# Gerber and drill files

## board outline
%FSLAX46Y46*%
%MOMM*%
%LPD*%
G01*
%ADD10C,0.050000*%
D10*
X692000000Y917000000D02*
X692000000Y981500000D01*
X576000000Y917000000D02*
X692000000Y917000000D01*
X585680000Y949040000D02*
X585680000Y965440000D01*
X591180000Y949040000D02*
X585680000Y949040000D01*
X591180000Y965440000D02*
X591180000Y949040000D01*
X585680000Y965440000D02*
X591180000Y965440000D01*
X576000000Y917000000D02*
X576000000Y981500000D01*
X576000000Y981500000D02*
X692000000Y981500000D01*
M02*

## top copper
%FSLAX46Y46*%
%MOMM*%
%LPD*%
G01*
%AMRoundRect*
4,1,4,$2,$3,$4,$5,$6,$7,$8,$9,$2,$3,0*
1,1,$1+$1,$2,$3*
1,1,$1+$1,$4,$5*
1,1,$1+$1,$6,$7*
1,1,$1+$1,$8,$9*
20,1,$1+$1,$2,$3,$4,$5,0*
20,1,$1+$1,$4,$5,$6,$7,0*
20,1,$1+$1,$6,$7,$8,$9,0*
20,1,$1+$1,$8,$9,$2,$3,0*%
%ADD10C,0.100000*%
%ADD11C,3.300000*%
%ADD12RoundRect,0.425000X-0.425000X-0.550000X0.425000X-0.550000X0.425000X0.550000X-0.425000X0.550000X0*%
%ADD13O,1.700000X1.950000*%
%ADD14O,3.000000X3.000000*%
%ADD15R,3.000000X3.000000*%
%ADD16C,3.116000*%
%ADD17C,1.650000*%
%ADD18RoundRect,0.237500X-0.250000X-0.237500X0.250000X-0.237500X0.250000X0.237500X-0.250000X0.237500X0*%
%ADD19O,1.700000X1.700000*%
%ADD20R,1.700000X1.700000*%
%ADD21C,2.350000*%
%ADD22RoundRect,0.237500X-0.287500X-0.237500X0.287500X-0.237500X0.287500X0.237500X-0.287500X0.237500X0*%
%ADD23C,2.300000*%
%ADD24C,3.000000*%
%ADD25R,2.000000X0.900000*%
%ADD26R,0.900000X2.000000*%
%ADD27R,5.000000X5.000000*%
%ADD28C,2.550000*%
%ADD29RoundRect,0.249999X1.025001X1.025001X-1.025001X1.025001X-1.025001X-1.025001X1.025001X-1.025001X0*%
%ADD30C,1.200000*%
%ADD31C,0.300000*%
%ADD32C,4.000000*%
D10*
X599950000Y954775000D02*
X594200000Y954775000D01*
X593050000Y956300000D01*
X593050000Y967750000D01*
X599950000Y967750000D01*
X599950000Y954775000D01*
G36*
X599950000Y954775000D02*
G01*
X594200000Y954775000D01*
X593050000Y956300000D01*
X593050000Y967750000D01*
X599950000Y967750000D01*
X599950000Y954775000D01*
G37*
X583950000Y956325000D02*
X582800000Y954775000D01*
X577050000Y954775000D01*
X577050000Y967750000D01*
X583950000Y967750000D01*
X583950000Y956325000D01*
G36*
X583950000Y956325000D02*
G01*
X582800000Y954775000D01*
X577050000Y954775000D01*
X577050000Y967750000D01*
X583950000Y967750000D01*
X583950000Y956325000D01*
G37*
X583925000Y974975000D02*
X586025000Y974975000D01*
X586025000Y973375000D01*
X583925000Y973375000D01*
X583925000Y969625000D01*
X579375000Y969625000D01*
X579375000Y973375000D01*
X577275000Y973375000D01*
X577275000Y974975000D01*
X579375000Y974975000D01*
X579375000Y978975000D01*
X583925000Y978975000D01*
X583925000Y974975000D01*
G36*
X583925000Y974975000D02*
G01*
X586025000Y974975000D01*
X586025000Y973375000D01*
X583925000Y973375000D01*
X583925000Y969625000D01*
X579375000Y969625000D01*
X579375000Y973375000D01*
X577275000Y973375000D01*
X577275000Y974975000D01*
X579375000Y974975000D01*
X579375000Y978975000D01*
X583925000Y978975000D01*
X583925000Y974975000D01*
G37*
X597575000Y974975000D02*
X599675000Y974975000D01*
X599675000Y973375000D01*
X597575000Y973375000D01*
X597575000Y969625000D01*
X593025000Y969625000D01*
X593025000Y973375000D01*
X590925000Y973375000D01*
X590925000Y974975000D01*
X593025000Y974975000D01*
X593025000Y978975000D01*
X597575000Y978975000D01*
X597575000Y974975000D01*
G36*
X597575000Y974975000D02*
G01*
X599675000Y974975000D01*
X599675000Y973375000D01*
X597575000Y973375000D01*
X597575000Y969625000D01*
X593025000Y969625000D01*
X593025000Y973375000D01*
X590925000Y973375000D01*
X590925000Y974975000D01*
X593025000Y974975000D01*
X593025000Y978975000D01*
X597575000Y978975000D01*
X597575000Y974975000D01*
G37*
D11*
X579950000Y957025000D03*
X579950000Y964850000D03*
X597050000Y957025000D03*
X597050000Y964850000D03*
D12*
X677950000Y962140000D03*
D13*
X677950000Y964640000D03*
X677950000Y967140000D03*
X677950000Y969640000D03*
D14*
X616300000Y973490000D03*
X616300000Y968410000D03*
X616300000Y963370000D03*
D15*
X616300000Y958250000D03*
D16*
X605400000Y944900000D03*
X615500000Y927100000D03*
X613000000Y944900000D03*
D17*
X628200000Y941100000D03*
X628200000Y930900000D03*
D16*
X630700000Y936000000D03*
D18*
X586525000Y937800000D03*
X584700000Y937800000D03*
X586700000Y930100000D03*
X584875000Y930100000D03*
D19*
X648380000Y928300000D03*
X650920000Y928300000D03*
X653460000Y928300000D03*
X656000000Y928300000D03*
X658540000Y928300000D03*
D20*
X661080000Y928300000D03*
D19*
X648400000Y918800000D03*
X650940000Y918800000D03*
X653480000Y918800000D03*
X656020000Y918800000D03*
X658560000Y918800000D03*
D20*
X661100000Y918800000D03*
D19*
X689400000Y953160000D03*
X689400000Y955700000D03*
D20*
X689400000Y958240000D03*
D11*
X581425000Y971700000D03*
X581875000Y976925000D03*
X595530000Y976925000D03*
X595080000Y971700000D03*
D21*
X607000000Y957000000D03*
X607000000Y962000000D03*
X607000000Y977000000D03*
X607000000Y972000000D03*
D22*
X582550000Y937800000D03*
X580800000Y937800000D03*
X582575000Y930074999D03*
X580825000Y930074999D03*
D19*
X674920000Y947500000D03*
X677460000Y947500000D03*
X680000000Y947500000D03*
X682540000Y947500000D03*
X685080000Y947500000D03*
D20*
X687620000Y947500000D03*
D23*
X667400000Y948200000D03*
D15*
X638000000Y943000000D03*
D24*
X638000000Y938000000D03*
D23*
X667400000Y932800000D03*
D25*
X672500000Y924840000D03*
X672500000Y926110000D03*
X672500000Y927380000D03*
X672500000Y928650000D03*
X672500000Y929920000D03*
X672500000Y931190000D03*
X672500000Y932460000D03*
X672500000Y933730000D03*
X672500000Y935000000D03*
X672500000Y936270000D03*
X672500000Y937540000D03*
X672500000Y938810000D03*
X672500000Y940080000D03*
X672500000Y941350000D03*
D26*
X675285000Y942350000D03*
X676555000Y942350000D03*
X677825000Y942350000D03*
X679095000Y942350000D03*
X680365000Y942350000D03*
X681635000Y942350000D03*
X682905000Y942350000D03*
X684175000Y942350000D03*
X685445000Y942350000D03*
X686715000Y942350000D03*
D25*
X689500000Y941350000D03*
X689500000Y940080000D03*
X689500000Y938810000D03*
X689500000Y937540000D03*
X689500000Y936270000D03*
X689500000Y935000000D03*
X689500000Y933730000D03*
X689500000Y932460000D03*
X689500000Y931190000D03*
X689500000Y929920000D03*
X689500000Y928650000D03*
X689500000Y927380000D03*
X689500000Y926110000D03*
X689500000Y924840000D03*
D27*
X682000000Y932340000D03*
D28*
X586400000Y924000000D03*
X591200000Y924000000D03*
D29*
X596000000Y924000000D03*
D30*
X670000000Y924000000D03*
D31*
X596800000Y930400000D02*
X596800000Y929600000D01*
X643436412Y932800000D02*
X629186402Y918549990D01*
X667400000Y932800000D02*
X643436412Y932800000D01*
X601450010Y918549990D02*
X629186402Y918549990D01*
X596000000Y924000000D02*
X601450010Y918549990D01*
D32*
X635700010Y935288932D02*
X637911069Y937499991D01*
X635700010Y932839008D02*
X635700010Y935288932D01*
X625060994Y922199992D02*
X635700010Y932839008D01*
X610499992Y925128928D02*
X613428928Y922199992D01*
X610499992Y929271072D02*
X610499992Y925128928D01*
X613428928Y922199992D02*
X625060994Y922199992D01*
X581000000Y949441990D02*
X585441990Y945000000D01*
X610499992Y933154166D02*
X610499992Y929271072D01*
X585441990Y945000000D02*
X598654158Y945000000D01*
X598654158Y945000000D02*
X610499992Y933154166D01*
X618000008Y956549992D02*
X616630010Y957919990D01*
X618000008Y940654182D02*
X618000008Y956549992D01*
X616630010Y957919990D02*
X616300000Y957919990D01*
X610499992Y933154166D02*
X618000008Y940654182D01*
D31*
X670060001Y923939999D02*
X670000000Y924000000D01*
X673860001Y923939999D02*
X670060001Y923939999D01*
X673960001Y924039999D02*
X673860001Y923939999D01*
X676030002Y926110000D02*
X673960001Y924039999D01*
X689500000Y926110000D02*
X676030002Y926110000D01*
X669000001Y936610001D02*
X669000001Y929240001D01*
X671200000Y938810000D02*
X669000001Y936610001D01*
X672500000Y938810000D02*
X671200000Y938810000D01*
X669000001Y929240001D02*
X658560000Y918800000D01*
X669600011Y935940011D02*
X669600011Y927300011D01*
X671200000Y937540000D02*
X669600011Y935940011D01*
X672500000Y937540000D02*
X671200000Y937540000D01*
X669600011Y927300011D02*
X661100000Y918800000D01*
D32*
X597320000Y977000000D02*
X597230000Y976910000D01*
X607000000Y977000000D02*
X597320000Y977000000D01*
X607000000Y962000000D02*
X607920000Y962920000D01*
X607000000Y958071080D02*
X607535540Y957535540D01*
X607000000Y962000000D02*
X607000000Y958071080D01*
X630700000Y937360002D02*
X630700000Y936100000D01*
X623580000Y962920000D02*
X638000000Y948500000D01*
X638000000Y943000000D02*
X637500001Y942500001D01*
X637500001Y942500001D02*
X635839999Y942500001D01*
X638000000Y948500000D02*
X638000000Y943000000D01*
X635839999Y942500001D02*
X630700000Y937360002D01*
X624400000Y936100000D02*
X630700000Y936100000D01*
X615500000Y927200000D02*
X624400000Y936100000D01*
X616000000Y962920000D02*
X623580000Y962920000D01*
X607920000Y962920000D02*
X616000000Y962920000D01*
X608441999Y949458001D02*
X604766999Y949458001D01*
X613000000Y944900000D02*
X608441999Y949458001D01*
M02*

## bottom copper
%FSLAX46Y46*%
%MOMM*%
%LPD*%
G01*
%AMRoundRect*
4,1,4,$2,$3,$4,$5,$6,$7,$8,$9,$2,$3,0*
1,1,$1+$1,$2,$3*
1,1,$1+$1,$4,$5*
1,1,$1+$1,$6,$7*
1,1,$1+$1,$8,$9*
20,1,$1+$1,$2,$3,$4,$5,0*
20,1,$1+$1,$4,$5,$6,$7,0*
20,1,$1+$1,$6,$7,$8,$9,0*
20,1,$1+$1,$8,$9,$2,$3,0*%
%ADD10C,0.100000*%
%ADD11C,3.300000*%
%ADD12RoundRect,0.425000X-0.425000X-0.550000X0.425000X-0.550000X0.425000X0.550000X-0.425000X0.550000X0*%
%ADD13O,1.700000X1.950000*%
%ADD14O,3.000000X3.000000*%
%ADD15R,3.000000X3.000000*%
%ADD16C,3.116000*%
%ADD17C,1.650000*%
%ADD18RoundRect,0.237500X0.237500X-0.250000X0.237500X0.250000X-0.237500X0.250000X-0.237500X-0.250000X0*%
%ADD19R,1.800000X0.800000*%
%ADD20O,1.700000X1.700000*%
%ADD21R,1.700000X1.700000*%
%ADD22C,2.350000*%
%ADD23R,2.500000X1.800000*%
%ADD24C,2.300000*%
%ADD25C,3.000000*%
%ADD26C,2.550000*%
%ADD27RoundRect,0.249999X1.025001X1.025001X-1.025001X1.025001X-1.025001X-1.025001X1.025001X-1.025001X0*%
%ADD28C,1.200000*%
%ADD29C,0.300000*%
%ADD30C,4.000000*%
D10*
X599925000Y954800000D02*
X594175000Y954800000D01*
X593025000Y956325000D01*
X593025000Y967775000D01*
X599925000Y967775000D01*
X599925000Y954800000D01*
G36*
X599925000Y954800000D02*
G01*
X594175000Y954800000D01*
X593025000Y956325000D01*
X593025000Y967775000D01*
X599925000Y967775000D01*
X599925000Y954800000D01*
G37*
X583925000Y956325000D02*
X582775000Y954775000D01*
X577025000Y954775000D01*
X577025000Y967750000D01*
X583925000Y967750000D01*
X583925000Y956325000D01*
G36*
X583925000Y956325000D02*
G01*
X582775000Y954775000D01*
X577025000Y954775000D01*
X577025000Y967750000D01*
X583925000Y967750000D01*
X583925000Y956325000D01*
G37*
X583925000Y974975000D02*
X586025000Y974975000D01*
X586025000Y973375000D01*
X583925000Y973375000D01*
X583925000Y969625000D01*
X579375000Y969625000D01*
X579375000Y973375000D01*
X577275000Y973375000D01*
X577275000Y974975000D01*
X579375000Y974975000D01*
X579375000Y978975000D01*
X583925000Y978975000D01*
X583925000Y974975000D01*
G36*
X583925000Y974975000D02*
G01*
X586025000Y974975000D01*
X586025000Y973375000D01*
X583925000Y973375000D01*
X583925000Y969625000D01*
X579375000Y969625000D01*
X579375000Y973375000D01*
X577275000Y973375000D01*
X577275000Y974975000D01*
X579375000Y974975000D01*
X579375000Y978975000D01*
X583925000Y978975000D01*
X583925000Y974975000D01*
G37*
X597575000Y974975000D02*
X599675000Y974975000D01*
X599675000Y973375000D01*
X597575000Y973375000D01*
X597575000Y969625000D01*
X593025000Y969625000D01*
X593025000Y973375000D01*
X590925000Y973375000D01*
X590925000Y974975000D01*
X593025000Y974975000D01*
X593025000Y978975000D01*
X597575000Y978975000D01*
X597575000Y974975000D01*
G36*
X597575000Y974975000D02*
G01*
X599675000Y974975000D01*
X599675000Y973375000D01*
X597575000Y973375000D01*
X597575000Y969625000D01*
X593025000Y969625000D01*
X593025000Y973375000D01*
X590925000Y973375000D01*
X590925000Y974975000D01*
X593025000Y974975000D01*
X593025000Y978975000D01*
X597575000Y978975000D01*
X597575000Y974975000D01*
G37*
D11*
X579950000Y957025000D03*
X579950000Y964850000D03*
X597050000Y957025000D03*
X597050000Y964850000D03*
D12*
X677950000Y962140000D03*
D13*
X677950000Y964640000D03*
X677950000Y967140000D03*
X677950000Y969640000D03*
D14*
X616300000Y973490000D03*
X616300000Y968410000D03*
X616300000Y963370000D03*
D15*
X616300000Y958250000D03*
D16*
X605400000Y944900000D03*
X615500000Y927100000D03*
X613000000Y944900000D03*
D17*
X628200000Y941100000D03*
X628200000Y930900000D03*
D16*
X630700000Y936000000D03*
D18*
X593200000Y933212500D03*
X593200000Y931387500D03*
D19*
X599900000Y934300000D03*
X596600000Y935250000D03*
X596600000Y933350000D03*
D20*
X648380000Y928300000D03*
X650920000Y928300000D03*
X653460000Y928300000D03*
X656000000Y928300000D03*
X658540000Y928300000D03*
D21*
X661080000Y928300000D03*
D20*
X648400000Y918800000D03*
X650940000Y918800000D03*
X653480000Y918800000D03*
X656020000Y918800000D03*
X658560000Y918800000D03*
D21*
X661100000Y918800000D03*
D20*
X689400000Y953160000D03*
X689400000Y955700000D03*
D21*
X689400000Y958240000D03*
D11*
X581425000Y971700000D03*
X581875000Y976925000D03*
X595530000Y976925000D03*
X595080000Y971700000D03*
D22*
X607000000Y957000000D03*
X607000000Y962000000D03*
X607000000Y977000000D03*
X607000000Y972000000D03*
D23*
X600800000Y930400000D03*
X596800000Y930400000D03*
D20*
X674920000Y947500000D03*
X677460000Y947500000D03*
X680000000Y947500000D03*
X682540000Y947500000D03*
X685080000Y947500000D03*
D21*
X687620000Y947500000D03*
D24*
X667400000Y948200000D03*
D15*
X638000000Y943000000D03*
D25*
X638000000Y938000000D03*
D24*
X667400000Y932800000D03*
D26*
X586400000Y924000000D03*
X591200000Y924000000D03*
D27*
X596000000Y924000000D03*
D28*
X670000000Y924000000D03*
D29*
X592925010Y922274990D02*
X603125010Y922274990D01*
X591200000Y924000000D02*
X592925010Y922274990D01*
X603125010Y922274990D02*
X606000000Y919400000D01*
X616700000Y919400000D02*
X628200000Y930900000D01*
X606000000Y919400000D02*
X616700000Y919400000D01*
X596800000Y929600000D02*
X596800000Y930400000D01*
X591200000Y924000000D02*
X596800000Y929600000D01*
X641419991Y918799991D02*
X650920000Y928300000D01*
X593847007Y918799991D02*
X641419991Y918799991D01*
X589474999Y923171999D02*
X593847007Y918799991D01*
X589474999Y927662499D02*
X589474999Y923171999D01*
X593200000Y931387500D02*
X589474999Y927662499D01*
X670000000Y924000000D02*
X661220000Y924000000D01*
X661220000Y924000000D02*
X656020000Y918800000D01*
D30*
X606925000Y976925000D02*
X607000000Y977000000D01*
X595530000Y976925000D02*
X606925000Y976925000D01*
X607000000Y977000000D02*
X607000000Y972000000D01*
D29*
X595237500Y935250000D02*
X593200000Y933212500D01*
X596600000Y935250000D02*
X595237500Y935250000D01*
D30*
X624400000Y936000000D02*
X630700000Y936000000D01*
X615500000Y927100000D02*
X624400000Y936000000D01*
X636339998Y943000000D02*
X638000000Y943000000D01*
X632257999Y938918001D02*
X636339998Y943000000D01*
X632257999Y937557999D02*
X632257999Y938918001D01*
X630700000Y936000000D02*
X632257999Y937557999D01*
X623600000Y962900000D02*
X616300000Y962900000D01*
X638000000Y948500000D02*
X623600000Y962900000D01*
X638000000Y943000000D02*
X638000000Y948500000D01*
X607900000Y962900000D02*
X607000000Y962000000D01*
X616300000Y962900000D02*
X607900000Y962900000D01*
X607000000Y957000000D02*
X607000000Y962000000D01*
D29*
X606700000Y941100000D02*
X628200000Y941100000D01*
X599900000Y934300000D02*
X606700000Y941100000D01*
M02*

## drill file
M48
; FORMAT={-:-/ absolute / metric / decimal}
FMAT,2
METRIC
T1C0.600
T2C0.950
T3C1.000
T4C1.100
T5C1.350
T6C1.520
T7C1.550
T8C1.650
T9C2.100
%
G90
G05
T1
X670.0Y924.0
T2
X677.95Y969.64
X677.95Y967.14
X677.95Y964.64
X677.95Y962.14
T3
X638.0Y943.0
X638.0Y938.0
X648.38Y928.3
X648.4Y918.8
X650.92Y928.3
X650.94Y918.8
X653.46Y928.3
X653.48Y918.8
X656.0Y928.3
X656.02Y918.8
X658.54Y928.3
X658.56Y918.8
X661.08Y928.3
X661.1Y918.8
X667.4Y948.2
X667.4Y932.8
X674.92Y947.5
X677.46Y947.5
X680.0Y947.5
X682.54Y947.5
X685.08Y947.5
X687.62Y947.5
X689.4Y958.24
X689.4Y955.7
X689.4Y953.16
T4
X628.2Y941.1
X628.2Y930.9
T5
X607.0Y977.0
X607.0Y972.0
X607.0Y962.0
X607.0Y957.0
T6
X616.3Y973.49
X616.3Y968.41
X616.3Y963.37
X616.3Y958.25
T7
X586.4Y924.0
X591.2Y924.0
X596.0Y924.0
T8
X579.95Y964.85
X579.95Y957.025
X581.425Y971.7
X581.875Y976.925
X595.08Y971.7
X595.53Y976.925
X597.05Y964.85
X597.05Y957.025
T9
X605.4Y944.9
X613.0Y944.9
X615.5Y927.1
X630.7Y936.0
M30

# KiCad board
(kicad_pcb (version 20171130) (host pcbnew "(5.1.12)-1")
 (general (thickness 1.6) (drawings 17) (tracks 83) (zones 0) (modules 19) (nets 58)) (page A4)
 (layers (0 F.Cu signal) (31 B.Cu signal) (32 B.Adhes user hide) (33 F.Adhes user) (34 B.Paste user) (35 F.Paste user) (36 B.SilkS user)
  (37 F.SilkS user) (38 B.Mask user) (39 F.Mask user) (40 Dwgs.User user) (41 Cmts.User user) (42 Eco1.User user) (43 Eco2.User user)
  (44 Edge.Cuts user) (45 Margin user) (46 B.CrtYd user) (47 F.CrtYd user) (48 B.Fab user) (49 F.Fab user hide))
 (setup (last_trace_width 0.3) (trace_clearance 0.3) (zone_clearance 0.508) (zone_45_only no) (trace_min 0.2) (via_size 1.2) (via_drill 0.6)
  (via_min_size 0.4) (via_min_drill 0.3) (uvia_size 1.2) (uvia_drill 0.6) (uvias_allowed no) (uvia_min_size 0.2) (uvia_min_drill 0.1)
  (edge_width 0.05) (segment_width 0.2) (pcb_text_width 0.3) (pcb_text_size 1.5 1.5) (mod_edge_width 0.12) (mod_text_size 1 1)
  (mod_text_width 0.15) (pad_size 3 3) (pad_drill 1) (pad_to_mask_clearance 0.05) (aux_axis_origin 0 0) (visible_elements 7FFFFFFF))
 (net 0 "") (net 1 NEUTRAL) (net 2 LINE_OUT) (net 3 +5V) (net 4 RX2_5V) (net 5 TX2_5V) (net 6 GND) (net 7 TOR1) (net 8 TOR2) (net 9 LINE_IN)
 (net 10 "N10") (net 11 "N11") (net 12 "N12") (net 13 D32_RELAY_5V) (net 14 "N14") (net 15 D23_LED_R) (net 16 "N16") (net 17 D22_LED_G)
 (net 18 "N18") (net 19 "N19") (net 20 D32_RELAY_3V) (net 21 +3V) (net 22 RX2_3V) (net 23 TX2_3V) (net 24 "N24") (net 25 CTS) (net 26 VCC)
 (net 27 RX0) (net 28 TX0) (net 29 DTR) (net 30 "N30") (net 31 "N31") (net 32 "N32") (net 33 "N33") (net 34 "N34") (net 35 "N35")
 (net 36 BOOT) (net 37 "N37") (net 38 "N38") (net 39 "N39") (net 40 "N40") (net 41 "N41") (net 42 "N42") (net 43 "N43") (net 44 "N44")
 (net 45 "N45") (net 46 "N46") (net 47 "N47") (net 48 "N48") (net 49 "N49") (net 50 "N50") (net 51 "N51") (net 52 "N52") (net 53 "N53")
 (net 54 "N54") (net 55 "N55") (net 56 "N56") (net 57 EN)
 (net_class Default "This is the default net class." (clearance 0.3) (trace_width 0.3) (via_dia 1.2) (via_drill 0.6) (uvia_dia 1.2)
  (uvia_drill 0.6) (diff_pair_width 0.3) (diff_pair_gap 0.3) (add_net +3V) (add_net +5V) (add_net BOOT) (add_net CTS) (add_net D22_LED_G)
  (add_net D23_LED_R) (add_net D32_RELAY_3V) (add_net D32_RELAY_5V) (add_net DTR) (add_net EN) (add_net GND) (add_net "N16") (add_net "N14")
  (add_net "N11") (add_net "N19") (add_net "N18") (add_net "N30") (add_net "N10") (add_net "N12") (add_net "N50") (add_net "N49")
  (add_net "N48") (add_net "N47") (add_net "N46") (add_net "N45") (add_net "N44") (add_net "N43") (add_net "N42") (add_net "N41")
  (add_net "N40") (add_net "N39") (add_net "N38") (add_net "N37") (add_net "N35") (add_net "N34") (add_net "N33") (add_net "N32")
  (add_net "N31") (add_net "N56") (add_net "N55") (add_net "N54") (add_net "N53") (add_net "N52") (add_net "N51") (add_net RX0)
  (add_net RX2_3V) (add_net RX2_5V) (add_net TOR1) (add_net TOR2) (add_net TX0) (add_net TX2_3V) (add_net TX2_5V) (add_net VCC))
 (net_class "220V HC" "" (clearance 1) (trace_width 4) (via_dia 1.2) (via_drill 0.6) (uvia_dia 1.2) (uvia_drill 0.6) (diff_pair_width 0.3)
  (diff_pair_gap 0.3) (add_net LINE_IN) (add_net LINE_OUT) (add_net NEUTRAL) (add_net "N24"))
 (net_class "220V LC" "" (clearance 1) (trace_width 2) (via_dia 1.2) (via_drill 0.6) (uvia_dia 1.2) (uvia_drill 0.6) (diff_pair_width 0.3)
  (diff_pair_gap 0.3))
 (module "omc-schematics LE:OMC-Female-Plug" (layer F.Cu) (at 588.5 -962.1)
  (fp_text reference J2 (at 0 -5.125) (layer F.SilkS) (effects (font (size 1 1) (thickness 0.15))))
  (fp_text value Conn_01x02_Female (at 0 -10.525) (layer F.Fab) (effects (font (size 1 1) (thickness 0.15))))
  (fp_poly (pts (xy 11.425 7.3) (xy 5.675 7.3) (xy 4.525 5.775) (xy 4.525 -5.675) (xy 11.425 -5.675)) (layer B.Cu) (width 0.1))
  (fp_poly (pts (xy 11.45 7.325) (xy 5.7 7.325) (xy 4.55 5.8) (xy 4.55 -5.65) (xy 11.45 -5.65)) (layer F.Cu) (width 0.1))
  (fp_poly (pts (xy -4.575 5.775) (xy -5.725 7.325) (xy -11.475 7.325) (xy -11.475 -5.65) (xy -4.575 -5.65)) (layer B.Cu) (width 0.1))
  (fp_poly (pts (xy -4.55 5.775) (xy -5.7 7.325) (xy -11.45 7.325) (xy -11.45 -5.65) (xy -4.55 -5.65)) (layer F.Cu) (width 0.1))
  (pad 1 thru_hole circle (at -8.55 5.075) (size 3.3 3.3) (drill 1.65) (layers *.Cu *.Mask) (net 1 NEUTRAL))
  (pad 1 thru_hole circle (at -8.55 -2.75) (size 3.3 3.3) (drill 1.65) (layers *.Cu *.Mask) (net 1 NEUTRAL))
  (pad 2 thru_hole circle (at 8.55 5.075) (size 3.3 3.3) (drill 1.65) (layers *.Cu *.Mask) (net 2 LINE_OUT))
  (pad 2 thru_hole circle (at 8.55 -2.75) (size 3.3 3.3) (drill 1.65) (layers *.Cu *.Mask) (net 2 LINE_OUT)))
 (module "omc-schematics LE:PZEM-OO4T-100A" (layer F.Cu) (at 649.18 -965.9)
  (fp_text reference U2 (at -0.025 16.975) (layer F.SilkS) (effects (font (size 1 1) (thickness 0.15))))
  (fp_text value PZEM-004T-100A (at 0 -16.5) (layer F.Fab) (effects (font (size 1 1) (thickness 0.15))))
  (pad 5 thru_hole roundrect (at 28.77 3.76) (size 1.7 1.95) (drill 0.95) (layers *.Cu *.Mask) (roundrect_rratio 0.25) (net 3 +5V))
  (pad 6 thru_hole oval (at 28.77 1.26) (size 1.7 1.95) (drill 0.95) (layers *.Cu *.Mask) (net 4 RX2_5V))
  (pad 7 thru_hole oval (at 28.77 -1.24) (size 1.7 1.95) (drill 0.95) (layers *.Cu *.Mask) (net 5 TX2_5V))
  (pad 8 thru_hole oval (at 28.77 -3.74) (size 1.7 1.95) (drill 0.95) (layers *.Cu *.Mask) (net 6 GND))
  (pad 4 thru_hole oval (at -32.88 -7.59) (size 3 3) (drill 1.52) (layers *.Cu *.Mask) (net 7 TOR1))
  (pad 3 thru_hole oval (at -32.88 -2.51) (size 3 3) (drill 1.52) (layers *.Cu *.Mask) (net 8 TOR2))
  (pad 2 thru_hole oval (at -32.88 2.53) (size 3 3) (drill 1.52) (layers *.Cu *.Mask) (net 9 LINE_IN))
  (pad 1 thru_hole rect (at -32.88 7.65) (size 3 3) (drill 1.52) (layers *.Cu *.Mask) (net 1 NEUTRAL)))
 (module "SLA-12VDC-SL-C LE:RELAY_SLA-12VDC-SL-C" (layer F.Cu) (at 613 -936 90)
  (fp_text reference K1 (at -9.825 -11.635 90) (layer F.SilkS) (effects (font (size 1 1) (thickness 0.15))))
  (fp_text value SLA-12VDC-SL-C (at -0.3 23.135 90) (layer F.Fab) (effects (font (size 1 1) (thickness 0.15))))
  (pad NC thru_hole circle (at 8.9 -7.6 90) (size 3.116 3.116) (drill 2.1) (layers *.Cu *.Mask) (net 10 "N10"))
  (pad COM2 thru_hole circle (at -8.9 2.5 90) (size 3.116 3.116) (drill 2.1) (layers *.Cu *.Mask) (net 9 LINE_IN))
  (pad NO thru_hole circle (at 8.9 0 90) (size 3.116 3.116) (drill 2.1) (layers *.Cu *.Mask) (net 2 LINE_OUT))
  (pad C2 thru_hole circle (at 5.1 15.2 90) (size 1.65 1.65) (drill 1.1) (layers *.Cu *.Mask) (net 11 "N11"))
  (pad C1 thru_hole circle (at -5.1 15.2 90) (size 1.65 1.65) (drill 1.1) (layers *.Cu *.Mask) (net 3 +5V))
  (pad COM1 thru_hole circle (at 0 17.7 90) (size 3.116 3.116) (drill 2.1) (layers *.Cu *.Mask) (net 9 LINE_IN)))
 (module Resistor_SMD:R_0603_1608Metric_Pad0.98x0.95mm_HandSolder (layer B.Cu) (at 593.2 -932.3 90)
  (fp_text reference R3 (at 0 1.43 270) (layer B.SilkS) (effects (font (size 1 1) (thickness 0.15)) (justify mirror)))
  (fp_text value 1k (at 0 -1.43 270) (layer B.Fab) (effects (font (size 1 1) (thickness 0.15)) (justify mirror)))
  (pad 2 smd roundrect (at 0.9125 0 90) (size 0.975 0.95) (layers B.Cu B.Paste B.Mask) (roundrect_rratio 0.25) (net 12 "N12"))
  (pad 1 smd roundrect (at -0.9125 0 90) (size 0.975 0.95) (layers B.Cu B.Paste B.Mask) (roundrect_rratio 0.25) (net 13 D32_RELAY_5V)))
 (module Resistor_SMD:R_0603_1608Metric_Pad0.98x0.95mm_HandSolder (layer F.Cu) (at 585.6125 -937.8)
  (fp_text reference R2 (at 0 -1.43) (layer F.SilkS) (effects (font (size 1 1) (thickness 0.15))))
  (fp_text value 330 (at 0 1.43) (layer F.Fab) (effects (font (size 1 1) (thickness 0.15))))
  (pad 2 smd roundrect (at 0.9125 0) (size 0.975 0.95) (layers F.Cu F.Paste F.Mask) (roundrect_rratio 0.25) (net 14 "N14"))
  (pad 1 smd roundrect (at -0.9125 0) (size 0.975 0.95) (layers F.Cu F.Paste F.Mask) (roundrect_rratio 0.25) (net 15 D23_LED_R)))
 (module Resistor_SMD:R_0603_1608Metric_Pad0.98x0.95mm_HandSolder (layer F.Cu) (at 585.7875 -930.1)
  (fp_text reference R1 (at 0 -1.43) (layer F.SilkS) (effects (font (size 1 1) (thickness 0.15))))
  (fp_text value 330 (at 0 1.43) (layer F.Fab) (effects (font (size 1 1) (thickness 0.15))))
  (pad 2 smd roundrect (at 0.9125 0) (size 0.975 0.95) (layers F.Cu F.Paste F.Mask) (roundrect_rratio 0.25) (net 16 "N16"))
  (pad 1 smd roundrect (at -0.9125 0) (size 0.975 0.95) (layers F.Cu F.Paste F.Mask) (roundrect_rratio 0.25) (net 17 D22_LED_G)))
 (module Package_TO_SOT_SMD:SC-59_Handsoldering (layer B.Cu) (at 598.25 -934.3)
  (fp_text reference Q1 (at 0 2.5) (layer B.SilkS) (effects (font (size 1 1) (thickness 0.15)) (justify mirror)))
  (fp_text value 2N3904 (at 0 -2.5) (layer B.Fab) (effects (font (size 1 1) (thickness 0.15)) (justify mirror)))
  (pad 3 smd rect (at 1.65 0) (size 1.8 0.8) (layers B.Cu B.Paste B.Mask) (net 11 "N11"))
  (pad 2 smd rect (at -1.65 -0.95) (size 1.8 0.8) (layers B.Cu B.Paste B.Mask) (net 12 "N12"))
  (pad 1 smd rect (at -1.65 0.95) (size 1.8 0.8) (layers B.Cu B.Paste B.Mask) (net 6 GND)))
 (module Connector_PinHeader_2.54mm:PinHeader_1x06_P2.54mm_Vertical (layer F.Cu) (at 661.08 -928.3 270)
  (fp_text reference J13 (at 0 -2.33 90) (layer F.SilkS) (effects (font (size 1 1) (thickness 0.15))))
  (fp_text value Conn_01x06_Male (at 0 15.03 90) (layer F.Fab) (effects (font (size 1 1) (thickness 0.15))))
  (pad 6 thru_hole oval (at 0 12.7 270) (size 1.7 1.7) (drill 1) (layers *.Cu *.Mask) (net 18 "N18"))
  (pad 5 thru_hole oval (at 0 10.16 270) (size 1.7 1.7) (drill 1) (layers *.Cu *.Mask) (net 13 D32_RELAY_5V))
  (pad 4 thru_hole oval (at 0 7.62 270) (size 1.7 1.7) (drill 1) (layers *.Cu *.Mask) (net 6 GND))
  (pad 3 thru_hole oval (at 0 5.08 270) (size 1.7 1.7) (drill 1) (layers *.Cu *.Mask) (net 3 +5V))
  (pad 2 thru_hole oval (at 0 2.54 270) (size 1.7 1.7) (drill 1) (layers *.Cu *.Mask) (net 5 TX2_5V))
  (pad 1 thru_hole rect (at 0 0 270) (size 1.7 1.7) (drill 1) (layers *.Cu *.Mask) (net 4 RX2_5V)))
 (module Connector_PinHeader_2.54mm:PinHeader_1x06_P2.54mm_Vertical (layer F.Cu) (at 661.1 -918.8 270)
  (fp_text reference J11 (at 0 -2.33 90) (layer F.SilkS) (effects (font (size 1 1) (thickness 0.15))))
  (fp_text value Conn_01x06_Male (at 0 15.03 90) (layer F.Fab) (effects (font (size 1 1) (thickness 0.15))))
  (pad 6 thru_hole oval (at 0 12.7 270) (size 1.7 1.7) (drill 1) (layers *.Cu *.Mask) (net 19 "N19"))
  (pad 5 thru_hole oval (at 0 10.16 270) (size 1.7 1.7) (drill 1) (layers *.Cu *.Mask) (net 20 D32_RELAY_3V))
  (pad 4 thru_hole oval (at 0 7.62 270) (size 1.7 1.7) (drill 1) (layers *.Cu *.Mask) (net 6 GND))
  (pad 3 thru_hole oval (at 0 5.08 270) (size 1.7 1.7) (drill 1) (layers *.Cu *.Mask) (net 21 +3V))
  (pad 2 thru_hole oval (at 0 2.54 270) (size 1.7 1.7) (drill 1) (layers *.Cu *.Mask) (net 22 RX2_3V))
  (pad 1 thru_hole rect (at 0 0 270) (size 1.7 1.7) (drill 1) (layers *.Cu *.Mask) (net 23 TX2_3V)))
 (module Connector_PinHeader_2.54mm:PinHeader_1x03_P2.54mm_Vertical (layer F.Cu) (at 689.4 -958.24)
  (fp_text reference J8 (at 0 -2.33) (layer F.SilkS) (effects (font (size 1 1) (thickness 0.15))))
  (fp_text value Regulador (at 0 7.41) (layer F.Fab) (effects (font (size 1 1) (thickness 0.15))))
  (pad 3 thru_hole oval (at 0 5.08) (size 1.7 1.7) (drill 1) (layers *.Cu *.Mask) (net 3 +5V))
  (pad 2 thru_hole oval (at 0 2.54) (size 1.7 1.7) (drill 1) (layers *.Cu *.Mask) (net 21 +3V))
  (pad 1 thru_hole rect (at 0 0) (size 1.7 1.7) (drill 1) (layers *.Cu *.Mask) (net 6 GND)))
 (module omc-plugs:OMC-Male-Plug (layer F.Cu) (at 581.6 -974)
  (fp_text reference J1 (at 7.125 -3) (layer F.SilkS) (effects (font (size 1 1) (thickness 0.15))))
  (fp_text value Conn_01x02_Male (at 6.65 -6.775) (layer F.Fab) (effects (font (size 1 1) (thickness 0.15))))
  (fp_poly
   (pts (xy 2.325 -0.975) (xy 4.425 -0.975) (xy 4.425 0.625) (xy 2.325 0.625) (xy 2.325 4.375) (xy -2.225 4.375) (xy -2.225 0.625)
    (xy -4.325 0.625) (xy -4.325 -0.975) (xy -2.225 -0.975) (xy -2.225 -4.975) (xy 2.325 -4.975))
   (layer F.Cu) (width 0.1))
  (fp_poly
   (pts (xy 2.325 -0.975) (xy 4.425 -0.975) (xy 4.425 0.625) (xy 2.325 0.625) (xy 2.325 4.375) (xy -2.225 4.375) (xy -2.225 0.625)
    (xy -4.325 0.625) (xy -4.325 -0.975) (xy -2.225 -0.975) (xy -2.225 -4.975) (xy 2.325 -4.975))
   (layer B.Cu) (width 0.1))
  (fp_poly
   (pts (xy 15.975 -0.975) (xy 18.075 -0.975) (xy 18.075 0.625) (xy 15.975 0.625) (xy 15.975 4.375) (xy 11.425 4.375) (xy 11.425 0.625)
    (xy 9.325 0.625) (xy 9.325 -0.975) (xy 11.425 -0.975) (xy 11.425 -4.975) (xy 15.975 -4.975))
   (layer B.Cu) (width 0.1))
  (fp_poly
   (pts (xy 15.975 -0.975) (xy 18.075 -0.975) (xy 18.075 0.625) (xy 15.975 0.625) (xy 15.975 4.375) (xy 11.425 4.375) (xy 11.425 0.625)
    (xy 9.325 0.625) (xy 9.325 -0.975) (xy 11.425 -0.975) (xy 11.425 -4.975) (xy 15.975 -4.975))
   (layer F.Cu) (width 0.1))
  (pad 1 thru_hole circle (at -0.175 2.3) (size 3.3 3.3) (drill 1.65) (layers *.Cu *.Mask) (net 1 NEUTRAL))
  (pad 1 thru_hole circle (at 0.275 -2.925 270) (size 3.3 3.3) (drill 1.65) (layers *.Cu *.Mask) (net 1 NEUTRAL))
  (pad 2 thru_hole circle (at 13.93 -2.925 270) (size 3.3 3.3) (drill 1.65) (layers *.Cu *.Mask) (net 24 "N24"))
  (pad 2 thru_hole circle (at 13.48 2.3) (size 3.3 3.3) (drill 1.65) (layers *.Cu *.Mask) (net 24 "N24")))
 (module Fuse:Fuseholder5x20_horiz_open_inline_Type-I (layer F.Cu) (at 607 -957 90)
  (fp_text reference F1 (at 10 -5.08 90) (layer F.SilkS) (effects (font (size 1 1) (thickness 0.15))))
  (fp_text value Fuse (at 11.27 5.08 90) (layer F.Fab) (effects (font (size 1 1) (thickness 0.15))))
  (pad 1 thru_hole circle (at 0 0 90) (size 2.35 2.35) (drill 1.35) (layers *.Cu *.Mask) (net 9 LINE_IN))
  (pad 1 thru_hole circle (at 5 0 90) (size 2.35 2.35) (drill 1.35) (layers *.Cu *.Mask) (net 9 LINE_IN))
  (pad 2 thru_hole circle (at 20 0 90) (size 2.35 2.35) (drill 1.35) (layers *.Cu *.Mask) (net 24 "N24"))
  (pad 2 thru_hole circle (at 15 0 90) (size 2.35 2.35) (drill 1.35) (layers *.Cu *.Mask) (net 24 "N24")))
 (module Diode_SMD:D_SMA (layer B.Cu) (at 598.8 -930.4)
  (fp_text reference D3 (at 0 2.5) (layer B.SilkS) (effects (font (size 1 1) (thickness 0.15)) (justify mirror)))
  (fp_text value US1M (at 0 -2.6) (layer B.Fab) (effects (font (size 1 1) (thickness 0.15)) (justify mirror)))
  (pad 2 smd rect (at 2 0) (size 2.5 1.8) (layers B.Cu B.Paste B.Mask) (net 11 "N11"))
  (pad 1 smd rect (at -2 0) (size 2.5 1.8) (layers B.Cu B.Paste B.Mask) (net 3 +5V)))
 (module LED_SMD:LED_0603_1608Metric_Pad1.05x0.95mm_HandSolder (layer F.Cu) (at 581.675 -937.8)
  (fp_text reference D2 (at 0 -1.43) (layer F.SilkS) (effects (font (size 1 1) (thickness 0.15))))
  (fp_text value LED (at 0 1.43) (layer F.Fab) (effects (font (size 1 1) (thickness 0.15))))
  (pad 2 smd roundrect (at 0.875 0) (size 1.05 0.95) (layers F.Cu F.Paste F.Mask) (roundrect_rratio 0.25) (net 14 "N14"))
  (pad 1 smd roundrect (at -0.875 0) (size 1.05 0.95) (layers F.Cu F.Paste F.Mask) (roundrect_rratio 0.25) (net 6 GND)))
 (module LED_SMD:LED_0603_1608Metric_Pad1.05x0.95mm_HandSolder (layer F.Cu) (at 581.7 -930.074999)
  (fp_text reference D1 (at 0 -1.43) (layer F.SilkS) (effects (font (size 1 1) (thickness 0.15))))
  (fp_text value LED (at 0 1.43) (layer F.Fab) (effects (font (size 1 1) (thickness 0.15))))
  (pad 2 smd roundrect (at 0.875 0) (size 1.05 0.95) (layers F.Cu F.Paste F.Mask) (roundrect_rratio 0.25) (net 16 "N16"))
  (pad 1 smd roundrect (at -0.875 0) (size 1.05 0.95) (layers F.Cu F.Paste F.Mask) (roundrect_rratio 0.25) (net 6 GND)))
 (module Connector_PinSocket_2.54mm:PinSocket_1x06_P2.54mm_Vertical (layer F.Cu) (at 687.62 -947.5 270)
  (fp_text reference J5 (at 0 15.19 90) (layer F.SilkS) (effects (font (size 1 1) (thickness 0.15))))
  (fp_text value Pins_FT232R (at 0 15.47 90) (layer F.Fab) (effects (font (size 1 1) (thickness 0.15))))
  (pad 6 thru_hole oval (at 0 12.7 270) (size 1.7 1.7) (drill 1) (layers *.Cu *.Mask) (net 6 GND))
  (pad 5 thru_hole oval (at 0 10.16 270) (size 1.7 1.7) (drill 1) (layers *.Cu *.Mask) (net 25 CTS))
  (pad 4 thru_hole oval (at 0 7.62 270) (size 1.7 1.7) (drill 1) (layers *.Cu *.Mask) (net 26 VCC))
  (pad 3 thru_hole oval (at 0 5.08 270) (size 1.7 1.7) (drill 1) (layers *.Cu *.Mask) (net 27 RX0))
  (pad 2 thru_hole oval (at 0 2.54 270) (size 1.7 1.7) (drill 1) (layers *.Cu *.Mask) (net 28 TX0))
  (pad 1 thru_hole rect (at 0 0 270) (size 1.7 1.7) (drill 1) (layers *.Cu *.Mask) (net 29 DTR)))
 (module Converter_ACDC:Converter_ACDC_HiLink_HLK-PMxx (layer F.Cu) (at 638 -943)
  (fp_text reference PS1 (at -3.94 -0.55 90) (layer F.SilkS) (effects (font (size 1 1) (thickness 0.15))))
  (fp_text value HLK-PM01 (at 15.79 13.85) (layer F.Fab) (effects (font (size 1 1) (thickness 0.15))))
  (pad 3 thru_hole circle (at 29.4 -5.2) (size 2.3 2.3) (drill 1) (layers *.Cu *.Mask) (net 6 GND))
  (pad 1 thru_hole rect (at 0 0) (size 3 3) (drill 1) (layers *.Cu *.Mask) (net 9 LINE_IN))
  (pad 2 thru_hole circle (at 0 5) (size 3 3) (drill 1) (layers *.Cu *.Mask) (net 1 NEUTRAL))
  (pad 4 thru_hole circle (at 29.4 10.2) (size 2.3 2.3) (drill 1) (layers *.Cu *.Mask) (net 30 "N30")))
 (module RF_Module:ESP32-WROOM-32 (layer F.Cu) (at 681 -933.095 180)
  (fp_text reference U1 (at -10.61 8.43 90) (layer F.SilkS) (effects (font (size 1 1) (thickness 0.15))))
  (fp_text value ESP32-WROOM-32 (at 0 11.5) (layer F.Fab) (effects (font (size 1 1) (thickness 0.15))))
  (pad 38 smd rect (at 8.5 -8.255 180) (size 2 0.9) (layers F.Cu F.Paste F.Mask) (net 6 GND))
  (pad 37 smd rect (at 8.5 -6.985 180) (size 2 0.9) (layers F.Cu F.Paste F.Mask) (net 15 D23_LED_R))
  (pad 36 smd rect (at 8.5 -5.715 180) (size 2 0.9) (layers F.Cu F.Paste F.Mask) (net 17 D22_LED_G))
  (pad 35 smd rect (at 8.5 -4.445 180) (size 2 0.9) (layers F.Cu F.Paste F.Mask) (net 28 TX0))
  (pad 34 smd rect (at 8.5 -3.175 180) (size 2 0.9) (layers F.Cu F.Paste F.Mask) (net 27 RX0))
  (pad 33 smd rect (at 8.5 -1.905 180) (size 2 0.9) (layers F.Cu F.Paste F.Mask) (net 20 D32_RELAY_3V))
  (pad 32 smd rect (at 8.5 -0.635 180) (size 2 0.9) (layers F.Cu F.Paste F.Mask) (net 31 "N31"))
  (pad 31 smd rect (at 8.5 0.635 180) (size 2 0.9) (layers F.Cu F.Paste F.Mask) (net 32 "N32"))
  (pad 30 smd rect (at 8.5 1.905 180) (size 2 0.9) (layers F.Cu F.Paste F.Mask) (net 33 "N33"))
  (pad 29 smd rect (at 8.5 3.175 180) (size 2 0.9) (layers F.Cu F.Paste F.Mask) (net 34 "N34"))
  (pad 28 smd rect (at 8.5 4.445 180) (size 2 0.9) (layers F.Cu F.Paste F.Mask) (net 23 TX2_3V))
  (pad 27 smd rect (at 8.5 5.715 180) (size 2 0.9) (layers F.Cu F.Paste F.Mask) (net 22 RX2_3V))
  (pad 26 smd rect (at 8.5 6.985 180) (size 2 0.9) (layers F.Cu F.Paste F.Mask) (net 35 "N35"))
  (pad 25 smd rect (at 8.5 8.255 180) (size 2 0.9) (layers F.Cu F.Paste F.Mask) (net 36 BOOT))
  (pad 24 smd rect (at 5.715 9.255 270) (size 2 0.9) (layers F.Cu F.Paste F.Mask) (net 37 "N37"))
  (pad 23 smd rect (at 4.445 9.255 270) (size 2 0.9) (layers F.Cu F.Paste F.Mask) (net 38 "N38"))
  (pad 22 smd rect (at 3.175 9.255 270) (size 2 0.9) (layers F.Cu F.Paste F.Mask) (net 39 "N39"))
  (pad 21 smd rect (at 1.905 9.255 270) (size 2 0.9) (layers F.Cu F.Paste F.Mask) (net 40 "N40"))
  (pad 20 smd rect (at 0.635 9.255 270) (size 2 0.9) (layers F.Cu F.Paste F.Mask) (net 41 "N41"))
  (pad 19 smd rect (at -0.635 9.255 270) (size 2 0.9) (layers F.Cu F.Paste F.Mask) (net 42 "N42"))
  (pad 18 smd rect (at -1.905 9.255 270) (size 2 0.9) (layers F.Cu F.Paste F.Mask) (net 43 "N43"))
  (pad 17 smd rect (at -3.175 9.255 270) (size 2 0.9) (layers F.Cu F.Paste F.Mask) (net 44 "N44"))
  (pad 16 smd rect (at -4.445 9.255 270) (size 2 0.9) (layers F.Cu F.Paste F.Mask) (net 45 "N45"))
  (pad 15 smd rect (at -5.715 9.255 270) (size 2 0.9) (layers F.Cu F.Paste F.Mask) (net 6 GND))
  (pad 14 smd rect (at -8.5 8.255 180) (size 2 0.9) (layers F.Cu F.Paste F.Mask) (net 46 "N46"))
  (pad 13 smd rect (at -8.5 6.985 180) (size 2 0.9) (layers F.Cu F.Paste F.Mask) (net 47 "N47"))
  (pad 12 smd rect (at -8.5 5.715 180) (size 2 0.9) (layers F.Cu F.Paste F.Mask) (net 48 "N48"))
  (pad 11 smd rect (at -8.5 4.445 180) (size 2 0.9) (layers F.Cu F.Paste F.Mask) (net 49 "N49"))
  (pad 10 smd rect (at -8.5 3.175 180) (size 2 0.9) (layers F.Cu F.Paste F.Mask) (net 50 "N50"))
  (pad 9 smd rect (at -8.5 1.905 180) (size 2 0.9) (layers F.Cu F.Paste F.Mask) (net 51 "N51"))
  (pad 8 smd rect (at -8.5 0.635 180) (size 2 0.9) (layers F.Cu F.Paste F.Mask) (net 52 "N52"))
  (pad 7 smd rect (at -8.5 -0.635 180) (size 2 0.9) (layers F.Cu F.Paste F.Mask) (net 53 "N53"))
  (pad 6 smd rect (at -8.5 -1.905 180) (size 2 0.9) (layers F.Cu F.Paste F.Mask) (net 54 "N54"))
  (pad 5 smd rect (at -8.5 -3.175 180) (size 2 0.9) (layers F.Cu F.Paste F.Mask) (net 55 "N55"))
  (pad 4 smd rect (at -8.5 -4.445 180) (size 2 0.9) (layers F.Cu F.Paste F.Mask) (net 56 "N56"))
  (pad 3 smd rect (at -8.5 -5.715 180) (size 2 0.9) (layers F.Cu F.Paste F.Mask) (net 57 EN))
  (pad 2 smd rect (at -8.5 -6.985 180) (size 2 0.9) (layers F.Cu F.Paste F.Mask) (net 21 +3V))
  (pad 1 smd rect (at -8.5 -8.255 180) (size 2 0.9) (layers F.Cu F.Paste F.Mask) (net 6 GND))
  (pad 39 smd rect (at -1 -0.755 180) (size 5 5) (layers F.Cu F.Paste F.Mask) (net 6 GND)))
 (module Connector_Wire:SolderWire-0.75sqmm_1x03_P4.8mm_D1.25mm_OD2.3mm (layer F.Cu) (at 596 -924 180)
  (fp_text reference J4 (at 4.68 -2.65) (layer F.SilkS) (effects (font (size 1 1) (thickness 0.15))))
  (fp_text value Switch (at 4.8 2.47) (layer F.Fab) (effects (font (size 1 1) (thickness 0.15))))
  (pad 3 thru_hole circle (at 9.6 0 180) (size 2.55 2.55) (drill 1.55) (layers *.Cu *.Mask) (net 6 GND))
  (pad 2 thru_hole circle (at 4.8 0 180) (size 2.55 2.55) (drill 1.55) (layers *.Cu *.Mask) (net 3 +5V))
  (pad 1 thru_hole roundrect (at 0 0 180) (size 2.55 2.55) (drill 1.55) (layers *.Cu *.Mask) (roundrect_rratio 0.09803882352941176)
   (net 30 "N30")))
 (gr_line (start 692 -917) (end 692 -981.5) (layer Edge.Cuts) (width 0.05))
 (gr_line (start 576 -917) (end 692 -917) (layer Edge.Cuts) (width 0.05))
 (gr_line (start 585.68 -949.04) (end 585.68 -965.44) (layer Edge.Cuts) (width 0.05))
 (gr_line (start 591.18 -949.04) (end 585.68 -949.04) (layer Edge.Cuts) (width 0.05))
 (gr_line (start 591.18 -965.44) (end 591.18 -949.04) (layer Edge.Cuts) (width 0.05))
 (gr_line (start 585.68 -965.44) (end 591.18 -965.44) (layer Edge.Cuts) (width 0.05))
 (gr_line (start 576 -917) (end 576 -981.5) (layer Edge.Cuts) (width 0.05))
 (gr_line (start 576 -981.5) (end 692 -981.5) (layer Edge.Cuts) (width 0.05))
 (segment (start 592.92501 -922.27499) (end 603.12501 -922.27499) (width 0.3) (layer B.Cu) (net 3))
 (segment (start 591.2 -924) (end 592.92501 -922.27499) (width 0.3) (layer B.Cu) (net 3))
 (segment (start 603.12501 -922.27499) (end 606 -919.4) (width 0.3) (layer B.Cu) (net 3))
 (segment (start 616.7 -919.4) (end 628.2 -930.9) (width 0.3) (layer B.Cu) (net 3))
 (segment (start 606 -919.4) (end 616.7 -919.4) (width 0.3) (layer B.Cu) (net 3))
 (segment (start 596.8 -930.4) (end 596.8 -929.6) (width 0.3) (layer F.Cu) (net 3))
 (segment (start 596.8 -929.6) (end 596.8 -930.4) (width 0.3) (layer B.Cu) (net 3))
 (segment (start 591.2 -924) (end 596.8 -929.6) (width 0.3) (layer B.Cu) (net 3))
 (segment (start 643.436412 -932.8) (end 629.186402 -918.54999) (width 0.3) (layer F.Cu) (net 30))
 (segment (start 667.4 -932.8) (end 643.436412 -932.8) (width 0.3) (layer F.Cu) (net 30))
 (segment (start 601.45001 -918.54999) (end 629.186402 -918.54999) (width 0.3) (layer F.Cu) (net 30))
 (segment (start 596 -924) (end 601.45001 -918.54999) (width 0.3) (layer F.Cu) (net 30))
 (segment (start 635.70001 -935.288932) (end 637.911069 -937.499991) (width 4) (layer F.Cu) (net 1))
 (segment (start 635.70001 -932.839008) (end 635.70001 -935.288932) (width 4) (layer F.Cu) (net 1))
 (segment (start 625.060994 -922.199992) (end 635.70001 -932.839008) (width 4) (layer F.Cu) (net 1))
 (segment (start 610.499992 -925.128928) (end 613.428928 -922.199992) (width 4) (layer F.Cu) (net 1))
 (segment (start 610.499992 -929.271072) (end 610.499992 -925.128928) (width 4) (layer F.Cu) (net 1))
 (segment (start 613.428928 -922.199992) (end 625.060994 -922.199992) (width 4) (layer F.Cu) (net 1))
 (segment (start 581 -949.44199) (end 585.44199 -945) (width 4) (layer F.Cu) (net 1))
 (segment (start 610.499992 -933.154166) (end 610.499992 -929.271072) (width 4) (layer F.Cu) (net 1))
 (segment (start 585.44199 -945) (end 598.654158 -945) (width 4) (layer F.Cu) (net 1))
 (segment (start 598.654158 -945) (end 610.499992 -933.154166) (width 4) (layer F.Cu) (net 1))
 (segment (start 618.000008 -956.549992) (end 616.63001 -957.91999) (width 4) (layer F.Cu) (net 1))
 (segment (start 618.000008 -940.654182) (end 618.000008 -956.549992) (width 4) (layer F.Cu) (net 1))
 (segment (start 616.63001 -957.91999) (end 616.3 -957.91999) (width 4) (layer F.Cu) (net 1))
 (segment (start 610.499992 -933.154166) (end 618.000008 -940.654182) (width 4) (layer F.Cu) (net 1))
 (segment (start 641.419991 -918.799991) (end 650.92 -928.3) (width 0.3) (layer B.Cu) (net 13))
 (segment (start 593.847007 -918.799991) (end 641.419991 -918.799991) (width 0.3) (layer B.Cu) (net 13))
 (segment (start 589.474999 -923.171999) (end 593.847007 -918.799991) (width 0.3) (layer B.Cu) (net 13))
 (segment (start 589.474999 -927.662499) (end 589.474999 -923.171999) (width 0.3) (layer B.Cu) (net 13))
 (segment (start 593.2 -931.3875) (end 589.474999 -927.662499) (width 0.3) (layer B.Cu) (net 13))
 (segment (start 670.060001 -923.939999) (end 670 -924) (width 0.3) (layer F.Cu) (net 21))
 (segment (start 673.860001 -923.939999) (end 670.060001 -923.939999) (width 0.3) (layer F.Cu) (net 21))
 (segment (start 673.960001 -924.039999) (end 673.860001 -923.939999) (width 0.3) (layer F.Cu) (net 21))
 (segment (start 676.030002 -926.11) (end 673.960001 -924.039999) (width 0.3) (layer F.Cu) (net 21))
 (segment (start 689.5 -926.11) (end 676.030002 -926.11) (width 0.3) (layer F.Cu) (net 21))
 (via (at 670 -924) (size 1.2) (drill 0.6) (layers F.Cu B.Cu) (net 21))
 (segment (start 670 -924) (end 661.22 -924) (width 0.3) (layer B.Cu) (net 21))
 (segment (start 661.22 -924) (end 656.02 -918.8) (width 0.3) (layer B.Cu) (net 21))
 (segment (start 669.000001 -936.610001) (end 669.000001 -929.240001) (width 0.3) (layer F.Cu) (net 22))
 (segment (start 671.2 -938.81) (end 669.000001 -936.610001) (width 0.3) (layer F.Cu) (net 22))
 (segment (start 672.5 -938.81) (end 671.2 -938.81) (width 0.3) (layer F.Cu) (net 22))
 (segment (start 669.000001 -929.240001) (end 658.56 -918.8) (width 0.3) (layer F.Cu) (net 22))
 (segment (start 669.600011 -935.940011) (end 669.600011 -927.300011) (width 0.3) (layer F.Cu) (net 23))
 (segment (start 671.2 -937.54) (end 669.600011 -935.940011) (width 0.3) (layer F.Cu) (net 23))
 (segment (start 672.5 -937.54) (end 671.2 -937.54) (width 0.3) (layer F.Cu) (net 23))
 (segment (start 669.600011 -927.300011) (end 661.1 -918.8) (width 0.3) (layer F.Cu) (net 23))
 (segment (start 597.32 -977) (end 597.23 -976.91) (width 4) (layer F.Cu) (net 24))
 (segment (start 607 -977) (end 597.32 -977) (width 4) (layer F.Cu) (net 24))
 (segment (start 606.925 -976.925) (end 607 -977) (width 4) (layer B.Cu) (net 24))
 (segment (start 595.53 -976.925) (end 606.925 -976.925) (width 4) (layer B.Cu) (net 24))
 (segment (start 607 -977) (end 607 -972) (width 4) (layer B.Cu) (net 24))
 (segment (start 595.2375 -935.25) (end 593.2 -933.2125) (width 0.3) (layer B.Cu) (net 12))
 (segment (start 596.6 -935.25) (end 595.2375 -935.25) (width 0.3) (layer B.Cu) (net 12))
 (segment (start 607 -962) (end 607.92 -962.92) (width 4) (layer F.Cu) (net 9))
 (segment (start 607 -958.07108) (end 607.53554 -957.53554) (width 4) (layer F.Cu) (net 9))
 (segment (start 607 -962) (end 607 -958.07108) (width 4) (layer F.Cu) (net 9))
 (segment (start 630.7 -937.360002) (end 630.7 -936.1) (width 4) (layer F.Cu) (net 9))
 (segment (start 623.58 -962.92) (end 638 -948.5) (width 4) (layer F.Cu) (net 9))
 (segment (start 638 -943) (end 637.500001 -942.500001) (width 4) (layer F.Cu) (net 9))
 (segment (start 637.500001 -942.500001) (end 635.839999 -942.500001) (width 4) (layer F.Cu) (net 9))
 (segment (start 638 -948.5) (end 638 -943) (width 4) (layer F.Cu) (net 9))
 (segment (start 635.839999 -942.500001) (end 630.7 -937.360002) (width 4) (layer F.Cu) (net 9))
 (segment (start 624.4 -936.1) (end 630.7 -936.1) (width 4) (layer F.Cu) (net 9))
 (segment (start 615.5 -927.2) (end 624.4 -936.1) (width 4) (layer F.Cu) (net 9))
 (segment (start 624.4 -936) (end 630.7 -936) (width 4) (layer B.Cu) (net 9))
 (segment (start 615.5 -927.1) (end 624.4 -936) (width 4) (layer B.Cu) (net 9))
 (segment (start 636.339998 -943) (end 638 -943) (width 4) (layer B.Cu) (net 9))
 (segment (start 632.257999 -938.918001) (end 636.339998 -943) (width 4) (layer B.Cu) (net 9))
 (segment (start 632.257999 -937.557999) (end 632.257999 -938.918001) (width 4) (layer B.Cu) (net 9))
 (segment (start 630.7 -936) (end 632.257999 -937.557999) (width 4) (layer B.Cu) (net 9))
 (segment (start 623.6 -962.9) (end 616.3 -962.9) (width 4) (layer B.Cu) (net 9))
 (segment (start 638 -948.5) (end 623.6 -962.9) (width 4) (layer B.Cu) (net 9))
 (segment (start 638 -943) (end 638 -948.5) (width 4) (layer B.Cu) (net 9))
 (segment (start 607.9 -962.9) (end 607 -962) (width 4) (layer B.Cu) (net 9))
 (segment (start 616.3 -962.9) (end 607.9 -962.9) (width 4) (layer B.Cu) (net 9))
 (segment (start 607 -957) (end 607 -962) (width 4) (layer B.Cu) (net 9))
 (segment (start 616 -962.92) (end 623.58 -962.92) (width 4) (layer F.Cu) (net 9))
 (segment (start 607.92 -962.92) (end 616 -962.92) (width 4) (layer F.Cu) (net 9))
 (segment (start 608.441999 -949.458001) (end 604.766999 -949.458001) (width 4) (layer F.Cu) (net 2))
 (segment (start 613 -944.9) (end 608.441999 -949.458001) (width 4) (layer F.Cu) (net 2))
 (segment (start 606.7 -941.1) (end 628.2 -941.1) (width 0.3) (layer B.Cu) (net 11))
 (segment (start 599.9 -934.3) (end 606.7 -941.1) (width 0.3) (layer B.Cu) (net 11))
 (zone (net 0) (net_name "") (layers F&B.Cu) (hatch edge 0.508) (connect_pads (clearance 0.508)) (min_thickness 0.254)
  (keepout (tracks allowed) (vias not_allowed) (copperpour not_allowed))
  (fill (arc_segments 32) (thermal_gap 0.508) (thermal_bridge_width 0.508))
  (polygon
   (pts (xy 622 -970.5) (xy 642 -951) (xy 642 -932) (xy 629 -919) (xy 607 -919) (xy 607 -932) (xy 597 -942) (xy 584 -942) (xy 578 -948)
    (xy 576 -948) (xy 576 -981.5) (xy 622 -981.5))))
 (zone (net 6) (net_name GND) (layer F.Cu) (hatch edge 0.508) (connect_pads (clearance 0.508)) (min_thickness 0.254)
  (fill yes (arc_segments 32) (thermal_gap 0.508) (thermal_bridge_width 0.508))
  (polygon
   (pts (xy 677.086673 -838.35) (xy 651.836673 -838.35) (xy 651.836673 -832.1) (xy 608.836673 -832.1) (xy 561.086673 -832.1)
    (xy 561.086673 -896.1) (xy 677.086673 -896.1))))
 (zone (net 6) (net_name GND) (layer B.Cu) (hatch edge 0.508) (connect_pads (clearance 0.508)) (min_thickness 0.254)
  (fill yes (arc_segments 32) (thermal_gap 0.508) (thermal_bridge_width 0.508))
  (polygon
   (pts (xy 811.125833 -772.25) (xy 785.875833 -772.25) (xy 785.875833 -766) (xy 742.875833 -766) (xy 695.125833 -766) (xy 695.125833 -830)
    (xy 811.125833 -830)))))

